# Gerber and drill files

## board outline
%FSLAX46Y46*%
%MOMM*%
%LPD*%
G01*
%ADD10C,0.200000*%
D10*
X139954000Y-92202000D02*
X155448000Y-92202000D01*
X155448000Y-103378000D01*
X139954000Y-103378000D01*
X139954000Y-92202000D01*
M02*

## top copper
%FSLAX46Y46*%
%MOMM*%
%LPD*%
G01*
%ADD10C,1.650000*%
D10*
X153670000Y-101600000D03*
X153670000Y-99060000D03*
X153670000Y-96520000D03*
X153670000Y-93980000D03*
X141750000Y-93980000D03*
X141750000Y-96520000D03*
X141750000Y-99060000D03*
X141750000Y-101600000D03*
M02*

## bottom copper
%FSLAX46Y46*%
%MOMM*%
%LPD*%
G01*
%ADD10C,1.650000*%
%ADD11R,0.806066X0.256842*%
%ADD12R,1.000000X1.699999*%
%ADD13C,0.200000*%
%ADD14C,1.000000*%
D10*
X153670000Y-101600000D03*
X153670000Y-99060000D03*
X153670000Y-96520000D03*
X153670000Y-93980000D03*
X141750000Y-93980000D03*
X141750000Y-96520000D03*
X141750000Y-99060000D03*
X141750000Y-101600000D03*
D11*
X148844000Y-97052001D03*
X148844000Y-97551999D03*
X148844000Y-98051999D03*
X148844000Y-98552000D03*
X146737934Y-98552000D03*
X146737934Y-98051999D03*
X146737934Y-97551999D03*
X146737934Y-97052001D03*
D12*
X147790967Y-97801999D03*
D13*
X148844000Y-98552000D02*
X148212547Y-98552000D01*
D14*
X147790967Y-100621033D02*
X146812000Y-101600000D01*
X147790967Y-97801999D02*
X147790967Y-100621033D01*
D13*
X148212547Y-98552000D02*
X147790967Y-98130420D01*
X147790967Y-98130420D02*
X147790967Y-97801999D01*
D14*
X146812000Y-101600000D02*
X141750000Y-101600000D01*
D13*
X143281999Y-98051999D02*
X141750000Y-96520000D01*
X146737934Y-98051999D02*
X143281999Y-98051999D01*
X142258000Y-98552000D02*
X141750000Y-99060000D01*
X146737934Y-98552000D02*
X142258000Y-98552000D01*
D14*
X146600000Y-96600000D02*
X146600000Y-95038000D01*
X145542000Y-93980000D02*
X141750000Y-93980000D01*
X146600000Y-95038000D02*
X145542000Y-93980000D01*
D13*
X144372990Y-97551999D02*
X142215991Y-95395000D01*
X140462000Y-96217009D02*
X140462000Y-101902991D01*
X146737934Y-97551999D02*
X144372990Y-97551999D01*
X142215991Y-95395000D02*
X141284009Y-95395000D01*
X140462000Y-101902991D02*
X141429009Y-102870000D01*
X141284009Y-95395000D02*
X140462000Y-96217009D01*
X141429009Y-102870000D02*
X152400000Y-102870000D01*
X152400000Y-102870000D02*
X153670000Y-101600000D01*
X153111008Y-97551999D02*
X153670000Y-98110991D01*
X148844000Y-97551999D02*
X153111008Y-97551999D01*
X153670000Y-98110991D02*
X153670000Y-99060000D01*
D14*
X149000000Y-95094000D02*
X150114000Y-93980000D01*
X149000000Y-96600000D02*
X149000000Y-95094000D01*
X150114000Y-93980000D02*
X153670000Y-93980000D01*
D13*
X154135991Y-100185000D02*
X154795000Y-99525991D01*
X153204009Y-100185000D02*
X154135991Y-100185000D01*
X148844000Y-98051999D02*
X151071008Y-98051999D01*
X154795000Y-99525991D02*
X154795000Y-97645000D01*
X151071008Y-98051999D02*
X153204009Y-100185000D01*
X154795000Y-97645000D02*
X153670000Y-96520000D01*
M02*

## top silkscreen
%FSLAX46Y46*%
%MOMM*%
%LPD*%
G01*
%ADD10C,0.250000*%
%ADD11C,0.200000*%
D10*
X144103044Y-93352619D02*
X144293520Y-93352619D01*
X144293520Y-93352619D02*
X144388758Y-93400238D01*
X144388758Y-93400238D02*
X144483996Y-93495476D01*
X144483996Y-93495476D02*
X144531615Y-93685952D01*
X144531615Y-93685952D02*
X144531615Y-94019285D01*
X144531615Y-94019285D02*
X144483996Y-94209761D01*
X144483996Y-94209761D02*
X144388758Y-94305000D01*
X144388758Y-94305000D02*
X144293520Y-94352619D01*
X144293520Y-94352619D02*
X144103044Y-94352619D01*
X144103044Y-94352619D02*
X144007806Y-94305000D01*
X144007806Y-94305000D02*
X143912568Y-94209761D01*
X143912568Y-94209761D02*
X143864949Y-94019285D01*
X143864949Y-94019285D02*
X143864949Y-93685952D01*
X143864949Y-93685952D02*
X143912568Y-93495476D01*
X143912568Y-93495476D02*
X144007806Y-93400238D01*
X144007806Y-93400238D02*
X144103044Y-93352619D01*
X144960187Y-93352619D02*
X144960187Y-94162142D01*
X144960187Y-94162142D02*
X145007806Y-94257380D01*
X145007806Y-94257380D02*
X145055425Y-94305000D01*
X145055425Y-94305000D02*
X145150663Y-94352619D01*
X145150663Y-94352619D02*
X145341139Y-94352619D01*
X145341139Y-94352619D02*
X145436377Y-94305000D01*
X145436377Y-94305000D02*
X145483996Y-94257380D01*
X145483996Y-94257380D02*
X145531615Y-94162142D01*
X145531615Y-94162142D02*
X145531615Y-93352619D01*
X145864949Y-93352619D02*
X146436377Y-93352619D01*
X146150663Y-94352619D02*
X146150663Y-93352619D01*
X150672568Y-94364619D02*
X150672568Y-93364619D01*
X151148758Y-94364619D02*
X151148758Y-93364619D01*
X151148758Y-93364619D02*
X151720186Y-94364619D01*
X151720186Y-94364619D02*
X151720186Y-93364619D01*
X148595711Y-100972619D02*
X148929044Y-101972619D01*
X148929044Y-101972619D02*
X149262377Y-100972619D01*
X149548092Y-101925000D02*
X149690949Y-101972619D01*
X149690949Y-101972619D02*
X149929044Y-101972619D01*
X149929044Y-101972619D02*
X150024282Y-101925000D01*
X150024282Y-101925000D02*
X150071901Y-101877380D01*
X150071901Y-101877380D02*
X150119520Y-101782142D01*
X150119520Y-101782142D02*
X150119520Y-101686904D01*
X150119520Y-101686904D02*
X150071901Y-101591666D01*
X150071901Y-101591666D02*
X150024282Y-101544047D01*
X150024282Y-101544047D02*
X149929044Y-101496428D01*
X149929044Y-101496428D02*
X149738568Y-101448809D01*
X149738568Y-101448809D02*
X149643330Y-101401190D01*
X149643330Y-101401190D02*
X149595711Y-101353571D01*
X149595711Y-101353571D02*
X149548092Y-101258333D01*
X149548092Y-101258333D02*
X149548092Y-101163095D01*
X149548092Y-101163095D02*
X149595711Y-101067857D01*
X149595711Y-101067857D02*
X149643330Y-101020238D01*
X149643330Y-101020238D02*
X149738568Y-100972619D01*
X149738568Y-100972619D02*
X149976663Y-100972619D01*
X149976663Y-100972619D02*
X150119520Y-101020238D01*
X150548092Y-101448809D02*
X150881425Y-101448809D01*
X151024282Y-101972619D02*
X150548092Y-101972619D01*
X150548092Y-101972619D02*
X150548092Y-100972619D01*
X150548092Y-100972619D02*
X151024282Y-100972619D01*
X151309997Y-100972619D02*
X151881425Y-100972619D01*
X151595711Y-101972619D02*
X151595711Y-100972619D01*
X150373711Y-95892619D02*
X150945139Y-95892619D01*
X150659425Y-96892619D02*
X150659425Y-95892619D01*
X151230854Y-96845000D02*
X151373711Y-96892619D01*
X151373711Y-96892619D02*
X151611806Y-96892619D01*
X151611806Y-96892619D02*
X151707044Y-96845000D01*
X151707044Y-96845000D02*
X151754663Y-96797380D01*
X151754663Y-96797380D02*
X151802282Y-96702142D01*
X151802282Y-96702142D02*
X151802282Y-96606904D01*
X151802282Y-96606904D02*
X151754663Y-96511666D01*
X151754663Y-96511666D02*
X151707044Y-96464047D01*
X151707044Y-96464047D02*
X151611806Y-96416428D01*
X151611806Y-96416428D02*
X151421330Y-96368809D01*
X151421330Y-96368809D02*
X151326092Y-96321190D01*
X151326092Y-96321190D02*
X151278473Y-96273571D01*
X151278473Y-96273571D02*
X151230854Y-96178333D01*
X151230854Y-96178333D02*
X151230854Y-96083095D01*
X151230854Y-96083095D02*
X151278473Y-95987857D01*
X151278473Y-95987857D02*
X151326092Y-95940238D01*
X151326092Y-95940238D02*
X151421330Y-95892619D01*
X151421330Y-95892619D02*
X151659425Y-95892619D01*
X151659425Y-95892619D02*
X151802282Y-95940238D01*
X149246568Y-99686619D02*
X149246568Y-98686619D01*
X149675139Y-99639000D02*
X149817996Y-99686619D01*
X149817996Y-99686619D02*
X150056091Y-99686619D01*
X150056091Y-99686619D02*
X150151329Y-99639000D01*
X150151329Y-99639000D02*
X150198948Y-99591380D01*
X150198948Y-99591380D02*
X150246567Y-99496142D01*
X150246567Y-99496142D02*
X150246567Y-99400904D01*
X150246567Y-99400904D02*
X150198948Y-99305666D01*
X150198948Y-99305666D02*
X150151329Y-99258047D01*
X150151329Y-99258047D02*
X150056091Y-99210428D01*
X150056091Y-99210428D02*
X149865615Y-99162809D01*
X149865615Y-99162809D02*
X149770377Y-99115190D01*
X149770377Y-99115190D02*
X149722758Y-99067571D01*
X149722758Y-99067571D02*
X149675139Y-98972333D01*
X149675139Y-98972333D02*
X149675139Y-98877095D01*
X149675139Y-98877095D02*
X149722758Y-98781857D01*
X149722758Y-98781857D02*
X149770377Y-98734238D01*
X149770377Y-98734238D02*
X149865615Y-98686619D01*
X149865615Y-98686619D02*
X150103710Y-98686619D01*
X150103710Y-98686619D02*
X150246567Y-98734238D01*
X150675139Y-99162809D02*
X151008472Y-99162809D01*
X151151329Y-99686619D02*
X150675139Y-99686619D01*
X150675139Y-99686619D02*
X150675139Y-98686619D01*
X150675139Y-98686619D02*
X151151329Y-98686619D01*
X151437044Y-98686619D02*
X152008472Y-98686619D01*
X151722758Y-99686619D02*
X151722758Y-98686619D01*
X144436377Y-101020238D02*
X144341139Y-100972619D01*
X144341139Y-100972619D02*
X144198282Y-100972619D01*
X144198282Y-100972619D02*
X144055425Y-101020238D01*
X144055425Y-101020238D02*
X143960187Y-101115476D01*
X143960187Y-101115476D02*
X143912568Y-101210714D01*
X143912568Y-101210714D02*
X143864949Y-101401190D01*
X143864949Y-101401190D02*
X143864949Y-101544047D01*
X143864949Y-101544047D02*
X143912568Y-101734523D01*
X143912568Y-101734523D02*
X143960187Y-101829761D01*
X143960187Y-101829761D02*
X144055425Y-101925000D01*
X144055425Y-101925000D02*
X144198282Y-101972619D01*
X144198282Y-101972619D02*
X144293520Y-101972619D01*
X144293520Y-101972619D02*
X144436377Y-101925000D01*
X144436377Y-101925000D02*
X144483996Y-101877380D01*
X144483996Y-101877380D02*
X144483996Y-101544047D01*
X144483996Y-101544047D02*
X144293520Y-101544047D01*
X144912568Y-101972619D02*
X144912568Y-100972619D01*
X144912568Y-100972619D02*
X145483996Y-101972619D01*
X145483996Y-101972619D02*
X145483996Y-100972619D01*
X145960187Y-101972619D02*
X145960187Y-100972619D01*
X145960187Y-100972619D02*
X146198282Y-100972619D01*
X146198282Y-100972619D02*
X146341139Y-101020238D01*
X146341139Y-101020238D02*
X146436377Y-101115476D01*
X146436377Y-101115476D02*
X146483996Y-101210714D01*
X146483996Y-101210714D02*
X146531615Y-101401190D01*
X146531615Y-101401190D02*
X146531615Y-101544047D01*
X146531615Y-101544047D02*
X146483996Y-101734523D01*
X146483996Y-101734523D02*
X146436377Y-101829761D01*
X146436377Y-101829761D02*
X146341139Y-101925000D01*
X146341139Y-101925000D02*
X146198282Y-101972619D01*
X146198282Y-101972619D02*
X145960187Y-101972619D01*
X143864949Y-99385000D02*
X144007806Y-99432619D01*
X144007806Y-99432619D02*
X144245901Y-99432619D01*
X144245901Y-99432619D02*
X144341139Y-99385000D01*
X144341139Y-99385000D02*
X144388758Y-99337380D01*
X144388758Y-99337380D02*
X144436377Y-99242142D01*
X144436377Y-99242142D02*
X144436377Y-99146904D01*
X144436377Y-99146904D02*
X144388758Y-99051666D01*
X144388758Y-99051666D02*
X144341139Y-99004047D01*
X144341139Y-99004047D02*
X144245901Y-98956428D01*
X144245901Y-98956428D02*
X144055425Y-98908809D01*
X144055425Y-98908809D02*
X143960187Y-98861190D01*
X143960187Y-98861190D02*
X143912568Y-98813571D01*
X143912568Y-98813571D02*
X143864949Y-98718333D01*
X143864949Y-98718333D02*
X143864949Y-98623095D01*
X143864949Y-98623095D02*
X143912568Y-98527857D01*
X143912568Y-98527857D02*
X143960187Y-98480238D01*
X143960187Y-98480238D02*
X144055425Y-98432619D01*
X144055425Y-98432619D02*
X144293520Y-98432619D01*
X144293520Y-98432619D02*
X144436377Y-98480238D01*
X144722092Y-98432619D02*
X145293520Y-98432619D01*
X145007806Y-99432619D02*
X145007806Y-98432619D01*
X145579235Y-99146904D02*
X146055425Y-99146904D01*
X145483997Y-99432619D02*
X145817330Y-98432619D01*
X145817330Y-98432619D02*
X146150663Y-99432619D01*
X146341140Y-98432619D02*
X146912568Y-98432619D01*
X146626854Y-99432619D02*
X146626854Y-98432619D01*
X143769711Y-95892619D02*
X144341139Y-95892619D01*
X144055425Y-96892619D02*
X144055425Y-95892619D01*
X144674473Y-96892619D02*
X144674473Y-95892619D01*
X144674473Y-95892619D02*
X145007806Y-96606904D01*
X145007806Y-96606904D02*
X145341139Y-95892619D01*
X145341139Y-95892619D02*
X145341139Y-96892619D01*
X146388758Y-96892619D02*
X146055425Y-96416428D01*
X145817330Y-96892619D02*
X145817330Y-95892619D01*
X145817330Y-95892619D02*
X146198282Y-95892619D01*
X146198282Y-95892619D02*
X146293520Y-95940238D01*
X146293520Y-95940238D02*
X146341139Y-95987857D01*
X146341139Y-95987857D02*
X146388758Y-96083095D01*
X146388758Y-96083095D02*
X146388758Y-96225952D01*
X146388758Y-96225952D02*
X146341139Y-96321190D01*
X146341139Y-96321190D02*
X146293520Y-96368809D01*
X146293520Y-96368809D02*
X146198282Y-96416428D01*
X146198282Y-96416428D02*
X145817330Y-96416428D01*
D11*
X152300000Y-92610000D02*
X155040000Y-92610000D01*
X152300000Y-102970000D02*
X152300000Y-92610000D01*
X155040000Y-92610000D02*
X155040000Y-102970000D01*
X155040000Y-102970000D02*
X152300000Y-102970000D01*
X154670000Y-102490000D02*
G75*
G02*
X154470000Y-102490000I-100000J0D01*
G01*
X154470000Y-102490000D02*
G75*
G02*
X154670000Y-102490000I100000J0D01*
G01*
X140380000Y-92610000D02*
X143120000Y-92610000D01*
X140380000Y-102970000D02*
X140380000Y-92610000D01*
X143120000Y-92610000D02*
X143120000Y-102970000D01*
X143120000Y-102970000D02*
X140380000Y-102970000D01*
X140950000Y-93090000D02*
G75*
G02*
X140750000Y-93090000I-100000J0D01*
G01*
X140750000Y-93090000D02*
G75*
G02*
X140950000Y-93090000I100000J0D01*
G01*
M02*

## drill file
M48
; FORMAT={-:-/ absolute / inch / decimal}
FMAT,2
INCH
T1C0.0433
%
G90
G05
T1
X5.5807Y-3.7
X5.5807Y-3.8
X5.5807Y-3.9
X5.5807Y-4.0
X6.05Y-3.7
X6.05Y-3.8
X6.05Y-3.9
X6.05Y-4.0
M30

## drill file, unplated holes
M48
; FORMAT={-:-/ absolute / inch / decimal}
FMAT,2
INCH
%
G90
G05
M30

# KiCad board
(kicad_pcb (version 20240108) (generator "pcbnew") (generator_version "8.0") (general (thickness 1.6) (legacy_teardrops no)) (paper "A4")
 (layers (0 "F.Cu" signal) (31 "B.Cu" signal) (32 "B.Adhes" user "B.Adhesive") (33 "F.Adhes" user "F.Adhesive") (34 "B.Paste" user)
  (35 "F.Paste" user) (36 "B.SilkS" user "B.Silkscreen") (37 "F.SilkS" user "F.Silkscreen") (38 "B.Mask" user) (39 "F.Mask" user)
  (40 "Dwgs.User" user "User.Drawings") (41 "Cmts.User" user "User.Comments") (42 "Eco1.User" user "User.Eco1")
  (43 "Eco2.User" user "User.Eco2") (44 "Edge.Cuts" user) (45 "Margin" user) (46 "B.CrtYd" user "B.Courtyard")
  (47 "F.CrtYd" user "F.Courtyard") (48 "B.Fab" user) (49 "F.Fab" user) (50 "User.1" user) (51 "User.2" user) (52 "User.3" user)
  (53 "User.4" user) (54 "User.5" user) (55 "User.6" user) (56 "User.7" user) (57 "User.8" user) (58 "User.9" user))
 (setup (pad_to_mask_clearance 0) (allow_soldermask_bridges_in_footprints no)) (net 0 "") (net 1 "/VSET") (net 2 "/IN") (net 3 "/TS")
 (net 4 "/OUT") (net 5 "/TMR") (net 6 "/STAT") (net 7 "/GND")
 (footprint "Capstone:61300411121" (layer "F.Cu") (at 153.67 97.79 90)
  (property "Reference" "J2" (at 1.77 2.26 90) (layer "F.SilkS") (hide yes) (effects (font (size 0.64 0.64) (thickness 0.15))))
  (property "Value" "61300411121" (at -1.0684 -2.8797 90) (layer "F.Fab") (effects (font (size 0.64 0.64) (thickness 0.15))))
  (fp_line (start 5.18 -1.37) (end 5.18 1.37) (stroke (width 0.2) (type solid)) (layer "F.SilkS"))
  (fp_line (start -5.18 -1.37) (end 5.18 -1.37) (stroke (width 0.2) (type solid)) (layer "F.SilkS"))
  (fp_line (start 5.18 1.37) (end -5.18 1.37) (stroke (width 0.2) (type solid)) (layer "F.SilkS"))
  (fp_line (start -5.18 1.37) (end -5.18 -1.37) (stroke (width 0.2) (type solid)) (layer "F.SilkS"))
  (fp_circle (center -4.7 0.9) (end -4.6 0.9) (stroke (width 0.2) (type solid)) (fill none) (layer "F.SilkS"))
  (pad "1" thru_hole circle (at -3.81 0 90) (size 1.65 1.65) (drill 1.1) (layers "*.Cu" "*.Mask") (remove_unused_layers no) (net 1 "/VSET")
   (solder_mask_margin 0.102))
  (pad "2" thru_hole circle (at -1.27 0 90) (size 1.65 1.65) (drill 1.1) (layers "*.Cu" "*.Mask") (remove_unused_layers no) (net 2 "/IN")
   (solder_mask_margin 0.102))
  (pad "3" thru_hole circle (at 1.27 0 90) (size 1.65 1.65) (drill 1.1) (layers "*.Cu" "*.Mask") (remove_unused_layers no) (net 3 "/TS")
   (solder_mask_margin 0.102))
  (pad "4" thru_hole circle (at 3.81 0 90) (size 1.65 1.65) (drill 1.1) (layers "*.Cu" "*.Mask") (remove_unused_layers no) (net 2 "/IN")
   (solder_mask_margin 0.102)))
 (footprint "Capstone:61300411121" (layer "F.Cu") (at 141.75 97.79 -90)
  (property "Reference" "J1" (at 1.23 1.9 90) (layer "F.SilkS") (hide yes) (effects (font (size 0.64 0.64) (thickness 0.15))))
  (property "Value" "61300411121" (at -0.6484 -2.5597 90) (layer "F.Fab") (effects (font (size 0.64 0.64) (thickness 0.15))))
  (fp_line (start -5.18 1.37) (end -5.18 -1.37) (stroke (width 0.2) (type solid)) (layer "F.SilkS"))
  (fp_line (start 5.18 1.37) (end -5.18 1.37) (stroke (width 0.2) (type solid)) (layer "F.SilkS"))
  (fp_line (start -5.18 -1.37) (end 5.18 -1.37) (stroke (width 0.2) (type solid)) (layer "F.SilkS"))
  (fp_line (start 5.18 -1.37) (end 5.18 1.37) (stroke (width 0.2) (type solid)) (layer "F.SilkS"))
  (fp_circle (center -4.7 0.9) (end -4.6 0.9) (stroke (width 0.2) (type solid)) (fill none) (layer "F.SilkS"))
  (pad "1" thru_hole circle (at -3.81 0 270) (size 1.65 1.65) (drill 1.1) (layers "*.Cu" "*.Mask") (remove_unused_layers no) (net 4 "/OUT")
   (solder_mask_margin 0.102))
  (pad "2" thru_hole circle (at -1.27 0 270) (size 1.65 1.65) (drill 1.1) (layers "*.Cu" "*.Mask") (remove_unused_layers no) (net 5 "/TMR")
   (solder_mask_margin 0.102))
  (pad "3" thru_hole circle (at 1.27 0 270) (size 1.65 1.65) (drill 1.1) (layers "*.Cu" "*.Mask") (remove_unused_layers no) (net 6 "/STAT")
   (solder_mask_margin 0.102))
  (pad "4" thru_hole circle (at 3.81 0 270) (size 1.65 1.65) (drill 1.1) (layers "*.Cu" "*.Mask") (remove_unused_layers no) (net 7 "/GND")
   (solder_mask_margin 0.102)))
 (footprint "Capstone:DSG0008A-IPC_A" (layer "B.Cu") (at 147.790967 97.801999 180)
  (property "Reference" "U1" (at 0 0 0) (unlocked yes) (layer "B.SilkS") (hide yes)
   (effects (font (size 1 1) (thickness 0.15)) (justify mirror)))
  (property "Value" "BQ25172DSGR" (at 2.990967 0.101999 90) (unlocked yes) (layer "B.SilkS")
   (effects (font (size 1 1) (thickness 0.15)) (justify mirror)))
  (pad "1" smd rect (at -1.053033 0.749998 180) (size 0.806066 0.256842) (layers "B.Cu" "B.Paste" "B.Mask") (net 2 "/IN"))
  (pad "2" smd rect (at -1.053033 0.25 180) (size 0.806066 0.256842) (layers "B.Cu" "B.Paste" "B.Mask") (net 2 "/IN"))
  (pad "3" smd rect (at -1.053033 -0.25 180) (size 0.806066 0.256842) (layers "B.Cu" "B.Paste" "B.Mask") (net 3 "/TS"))
  (pad "4" smd rect (at -1.053033 -0.750001 180) (size 0.806066 0.256842) (layers "B.Cu" "B.Paste" "B.Mask") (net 7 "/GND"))
  (pad "5" smd rect (at 1.053033 -0.750001 180) (size 0.806066 0.256842) (layers "B.Cu" "B.Paste" "B.Mask") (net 6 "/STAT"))
  (pad "6" smd rect (at 1.053033 -0.25 180) (size 0.806066 0.256842) (layers "B.Cu" "B.Paste" "B.Mask") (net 5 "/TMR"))
  (pad "7" smd rect (at 1.053033 0.25 180) (size 0.806066 0.256842) (layers "B.Cu" "B.Paste" "B.Mask") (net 1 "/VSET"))
  (pad "8" smd rect (at 1.053033 0.749998 180) (size 0.806066 0.256842) (layers "B.Cu" "B.Paste" "B.Mask") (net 4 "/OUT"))
  (pad "9" smd rect (at 0 0 180) (size 1 1.699999) (layers "B.Cu" "B.Mask") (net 7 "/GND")))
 (gr_rect (start 139.954 92.202) (end 155.448 103.378) (stroke (width 0.2) (type default)) (fill none) (layer "Edge.Cuts"))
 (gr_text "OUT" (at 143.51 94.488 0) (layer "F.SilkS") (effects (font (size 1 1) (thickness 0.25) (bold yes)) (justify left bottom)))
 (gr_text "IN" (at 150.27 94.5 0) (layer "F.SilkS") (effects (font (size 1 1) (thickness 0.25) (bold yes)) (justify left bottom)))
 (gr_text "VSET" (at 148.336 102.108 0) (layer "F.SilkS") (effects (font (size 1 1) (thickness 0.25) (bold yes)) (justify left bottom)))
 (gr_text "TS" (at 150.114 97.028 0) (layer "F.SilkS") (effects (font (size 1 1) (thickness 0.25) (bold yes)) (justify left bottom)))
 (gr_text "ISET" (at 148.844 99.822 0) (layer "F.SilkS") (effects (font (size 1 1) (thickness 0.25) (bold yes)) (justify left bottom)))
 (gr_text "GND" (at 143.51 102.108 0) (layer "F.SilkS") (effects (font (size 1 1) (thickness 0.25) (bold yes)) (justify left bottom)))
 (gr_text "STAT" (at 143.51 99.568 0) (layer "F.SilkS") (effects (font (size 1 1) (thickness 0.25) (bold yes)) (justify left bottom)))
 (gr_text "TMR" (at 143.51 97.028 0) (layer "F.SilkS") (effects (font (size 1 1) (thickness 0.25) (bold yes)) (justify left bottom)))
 (segment (start 148.844 98.552) (end 148.212547 98.552) (width 0.2) (layer "B.Cu") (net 7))
 (segment (start 147.790967 100.621033) (end 146.812 101.6) (width 1) (layer "B.Cu") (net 7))
 (segment (start 147.790967 97.801999) (end 147.790967 100.621033) (width 1) (layer "B.Cu") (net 7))
 (segment (start 148.212547 98.552) (end 147.790967 98.13042) (width 0.2) (layer "B.Cu") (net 7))
 (segment (start 147.790967 98.13042) (end 147.790967 97.801999) (width 0.2) (layer "B.Cu") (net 7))
 (segment (start 146.812 101.6) (end 141.75 101.6) (width 1) (layer "B.Cu") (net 7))
 (segment (start 143.281999 98.051999) (end 141.75 96.52) (width 0.2) (layer "B.Cu") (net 5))
 (segment (start 146.737934 98.051999) (end 143.281999 98.051999) (width 0.2) (layer "B.Cu") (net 5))
 (segment (start 142.258 98.552) (end 141.75 99.06) (width 0.2) (layer "B.Cu") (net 6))
 (segment (start 146.737934 98.552) (end 142.258 98.552) (width 0.2) (layer "B.Cu") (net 6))
 (segment (start 146.6 96.6) (end 146.6 95.038) (width 1) (layer "B.Cu") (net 4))
 (segment (start 145.542 93.98) (end 141.75 93.98) (width 1) (layer "B.Cu") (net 4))
 (segment (start 146.6 95.038) (end 145.542 93.98) (width 1) (layer "B.Cu") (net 4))
 (segment (start 144.37299 97.551999) (end 142.215991 95.395) (width 0.2) (layer "B.Cu") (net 1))
 (segment (start 140.462 96.217009) (end 140.462 101.902991) (width 0.2) (layer "B.Cu") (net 1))
 (segment (start 146.737934 97.551999) (end 144.37299 97.551999) (width 0.2) (layer "B.Cu") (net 1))
 (segment (start 142.215991 95.395) (end 141.284009 95.395) (width 0.2) (layer "B.Cu") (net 1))
 (segment (start 140.462 101.902991) (end 141.429009 102.87) (width 0.2) (layer "B.Cu") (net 1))
 (segment (start 141.284009 95.395) (end 140.462 96.217009) (width 0.2) (layer "B.Cu") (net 1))
 (segment (start 141.429009 102.87) (end 152.4 102.87) (width 0.2) (layer "B.Cu") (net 1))
 (segment (start 152.4 102.87) (end 153.67 101.6) (width 0.2) (layer "B.Cu") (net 1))
 (segment (start 153.111008 97.551999) (end 153.67 98.110991) (width 0.2) (layer "B.Cu") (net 2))
 (segment (start 148.844 97.551999) (end 153.111008 97.551999) (width 0.2) (layer "B.Cu") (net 2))
 (segment (start 153.67 98.110991) (end 153.67 99.06) (width 0.2) (layer "B.Cu") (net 2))
 (segment (start 149 95.094) (end 150.114 93.98) (width 1) (layer "B.Cu") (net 2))
 (segment (start 149 96.6) (end 149 95.094) (width 1) (layer "B.Cu") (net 2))
 (segment (start 150.114 93.98) (end 153.67 93.98) (width 1) (layer "B.Cu") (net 2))
 (segment (start 154.135991 100.185) (end 154.795 99.525991) (width 0.2) (layer "B.Cu") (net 3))
 (segment (start 153.204009 100.185) (end 154.135991 100.185) (width 0.2) (layer "B.Cu") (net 3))
 (segment (start 148.844 98.051999) (end 151.071008 98.051999) (width 0.2) (layer "B.Cu") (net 3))
 (segment (start 154.795 99.525991) (end 154.795 97.645) (width 0.2) (layer "B.Cu") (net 3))
 (segment (start 151.071008 98.051999) (end 153.204009 100.185) (width 0.2) (layer "B.Cu") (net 3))
 (segment (start 154.795 97.645) (end 153.67 96.52) (width 0.2) (layer "B.Cu") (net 3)))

